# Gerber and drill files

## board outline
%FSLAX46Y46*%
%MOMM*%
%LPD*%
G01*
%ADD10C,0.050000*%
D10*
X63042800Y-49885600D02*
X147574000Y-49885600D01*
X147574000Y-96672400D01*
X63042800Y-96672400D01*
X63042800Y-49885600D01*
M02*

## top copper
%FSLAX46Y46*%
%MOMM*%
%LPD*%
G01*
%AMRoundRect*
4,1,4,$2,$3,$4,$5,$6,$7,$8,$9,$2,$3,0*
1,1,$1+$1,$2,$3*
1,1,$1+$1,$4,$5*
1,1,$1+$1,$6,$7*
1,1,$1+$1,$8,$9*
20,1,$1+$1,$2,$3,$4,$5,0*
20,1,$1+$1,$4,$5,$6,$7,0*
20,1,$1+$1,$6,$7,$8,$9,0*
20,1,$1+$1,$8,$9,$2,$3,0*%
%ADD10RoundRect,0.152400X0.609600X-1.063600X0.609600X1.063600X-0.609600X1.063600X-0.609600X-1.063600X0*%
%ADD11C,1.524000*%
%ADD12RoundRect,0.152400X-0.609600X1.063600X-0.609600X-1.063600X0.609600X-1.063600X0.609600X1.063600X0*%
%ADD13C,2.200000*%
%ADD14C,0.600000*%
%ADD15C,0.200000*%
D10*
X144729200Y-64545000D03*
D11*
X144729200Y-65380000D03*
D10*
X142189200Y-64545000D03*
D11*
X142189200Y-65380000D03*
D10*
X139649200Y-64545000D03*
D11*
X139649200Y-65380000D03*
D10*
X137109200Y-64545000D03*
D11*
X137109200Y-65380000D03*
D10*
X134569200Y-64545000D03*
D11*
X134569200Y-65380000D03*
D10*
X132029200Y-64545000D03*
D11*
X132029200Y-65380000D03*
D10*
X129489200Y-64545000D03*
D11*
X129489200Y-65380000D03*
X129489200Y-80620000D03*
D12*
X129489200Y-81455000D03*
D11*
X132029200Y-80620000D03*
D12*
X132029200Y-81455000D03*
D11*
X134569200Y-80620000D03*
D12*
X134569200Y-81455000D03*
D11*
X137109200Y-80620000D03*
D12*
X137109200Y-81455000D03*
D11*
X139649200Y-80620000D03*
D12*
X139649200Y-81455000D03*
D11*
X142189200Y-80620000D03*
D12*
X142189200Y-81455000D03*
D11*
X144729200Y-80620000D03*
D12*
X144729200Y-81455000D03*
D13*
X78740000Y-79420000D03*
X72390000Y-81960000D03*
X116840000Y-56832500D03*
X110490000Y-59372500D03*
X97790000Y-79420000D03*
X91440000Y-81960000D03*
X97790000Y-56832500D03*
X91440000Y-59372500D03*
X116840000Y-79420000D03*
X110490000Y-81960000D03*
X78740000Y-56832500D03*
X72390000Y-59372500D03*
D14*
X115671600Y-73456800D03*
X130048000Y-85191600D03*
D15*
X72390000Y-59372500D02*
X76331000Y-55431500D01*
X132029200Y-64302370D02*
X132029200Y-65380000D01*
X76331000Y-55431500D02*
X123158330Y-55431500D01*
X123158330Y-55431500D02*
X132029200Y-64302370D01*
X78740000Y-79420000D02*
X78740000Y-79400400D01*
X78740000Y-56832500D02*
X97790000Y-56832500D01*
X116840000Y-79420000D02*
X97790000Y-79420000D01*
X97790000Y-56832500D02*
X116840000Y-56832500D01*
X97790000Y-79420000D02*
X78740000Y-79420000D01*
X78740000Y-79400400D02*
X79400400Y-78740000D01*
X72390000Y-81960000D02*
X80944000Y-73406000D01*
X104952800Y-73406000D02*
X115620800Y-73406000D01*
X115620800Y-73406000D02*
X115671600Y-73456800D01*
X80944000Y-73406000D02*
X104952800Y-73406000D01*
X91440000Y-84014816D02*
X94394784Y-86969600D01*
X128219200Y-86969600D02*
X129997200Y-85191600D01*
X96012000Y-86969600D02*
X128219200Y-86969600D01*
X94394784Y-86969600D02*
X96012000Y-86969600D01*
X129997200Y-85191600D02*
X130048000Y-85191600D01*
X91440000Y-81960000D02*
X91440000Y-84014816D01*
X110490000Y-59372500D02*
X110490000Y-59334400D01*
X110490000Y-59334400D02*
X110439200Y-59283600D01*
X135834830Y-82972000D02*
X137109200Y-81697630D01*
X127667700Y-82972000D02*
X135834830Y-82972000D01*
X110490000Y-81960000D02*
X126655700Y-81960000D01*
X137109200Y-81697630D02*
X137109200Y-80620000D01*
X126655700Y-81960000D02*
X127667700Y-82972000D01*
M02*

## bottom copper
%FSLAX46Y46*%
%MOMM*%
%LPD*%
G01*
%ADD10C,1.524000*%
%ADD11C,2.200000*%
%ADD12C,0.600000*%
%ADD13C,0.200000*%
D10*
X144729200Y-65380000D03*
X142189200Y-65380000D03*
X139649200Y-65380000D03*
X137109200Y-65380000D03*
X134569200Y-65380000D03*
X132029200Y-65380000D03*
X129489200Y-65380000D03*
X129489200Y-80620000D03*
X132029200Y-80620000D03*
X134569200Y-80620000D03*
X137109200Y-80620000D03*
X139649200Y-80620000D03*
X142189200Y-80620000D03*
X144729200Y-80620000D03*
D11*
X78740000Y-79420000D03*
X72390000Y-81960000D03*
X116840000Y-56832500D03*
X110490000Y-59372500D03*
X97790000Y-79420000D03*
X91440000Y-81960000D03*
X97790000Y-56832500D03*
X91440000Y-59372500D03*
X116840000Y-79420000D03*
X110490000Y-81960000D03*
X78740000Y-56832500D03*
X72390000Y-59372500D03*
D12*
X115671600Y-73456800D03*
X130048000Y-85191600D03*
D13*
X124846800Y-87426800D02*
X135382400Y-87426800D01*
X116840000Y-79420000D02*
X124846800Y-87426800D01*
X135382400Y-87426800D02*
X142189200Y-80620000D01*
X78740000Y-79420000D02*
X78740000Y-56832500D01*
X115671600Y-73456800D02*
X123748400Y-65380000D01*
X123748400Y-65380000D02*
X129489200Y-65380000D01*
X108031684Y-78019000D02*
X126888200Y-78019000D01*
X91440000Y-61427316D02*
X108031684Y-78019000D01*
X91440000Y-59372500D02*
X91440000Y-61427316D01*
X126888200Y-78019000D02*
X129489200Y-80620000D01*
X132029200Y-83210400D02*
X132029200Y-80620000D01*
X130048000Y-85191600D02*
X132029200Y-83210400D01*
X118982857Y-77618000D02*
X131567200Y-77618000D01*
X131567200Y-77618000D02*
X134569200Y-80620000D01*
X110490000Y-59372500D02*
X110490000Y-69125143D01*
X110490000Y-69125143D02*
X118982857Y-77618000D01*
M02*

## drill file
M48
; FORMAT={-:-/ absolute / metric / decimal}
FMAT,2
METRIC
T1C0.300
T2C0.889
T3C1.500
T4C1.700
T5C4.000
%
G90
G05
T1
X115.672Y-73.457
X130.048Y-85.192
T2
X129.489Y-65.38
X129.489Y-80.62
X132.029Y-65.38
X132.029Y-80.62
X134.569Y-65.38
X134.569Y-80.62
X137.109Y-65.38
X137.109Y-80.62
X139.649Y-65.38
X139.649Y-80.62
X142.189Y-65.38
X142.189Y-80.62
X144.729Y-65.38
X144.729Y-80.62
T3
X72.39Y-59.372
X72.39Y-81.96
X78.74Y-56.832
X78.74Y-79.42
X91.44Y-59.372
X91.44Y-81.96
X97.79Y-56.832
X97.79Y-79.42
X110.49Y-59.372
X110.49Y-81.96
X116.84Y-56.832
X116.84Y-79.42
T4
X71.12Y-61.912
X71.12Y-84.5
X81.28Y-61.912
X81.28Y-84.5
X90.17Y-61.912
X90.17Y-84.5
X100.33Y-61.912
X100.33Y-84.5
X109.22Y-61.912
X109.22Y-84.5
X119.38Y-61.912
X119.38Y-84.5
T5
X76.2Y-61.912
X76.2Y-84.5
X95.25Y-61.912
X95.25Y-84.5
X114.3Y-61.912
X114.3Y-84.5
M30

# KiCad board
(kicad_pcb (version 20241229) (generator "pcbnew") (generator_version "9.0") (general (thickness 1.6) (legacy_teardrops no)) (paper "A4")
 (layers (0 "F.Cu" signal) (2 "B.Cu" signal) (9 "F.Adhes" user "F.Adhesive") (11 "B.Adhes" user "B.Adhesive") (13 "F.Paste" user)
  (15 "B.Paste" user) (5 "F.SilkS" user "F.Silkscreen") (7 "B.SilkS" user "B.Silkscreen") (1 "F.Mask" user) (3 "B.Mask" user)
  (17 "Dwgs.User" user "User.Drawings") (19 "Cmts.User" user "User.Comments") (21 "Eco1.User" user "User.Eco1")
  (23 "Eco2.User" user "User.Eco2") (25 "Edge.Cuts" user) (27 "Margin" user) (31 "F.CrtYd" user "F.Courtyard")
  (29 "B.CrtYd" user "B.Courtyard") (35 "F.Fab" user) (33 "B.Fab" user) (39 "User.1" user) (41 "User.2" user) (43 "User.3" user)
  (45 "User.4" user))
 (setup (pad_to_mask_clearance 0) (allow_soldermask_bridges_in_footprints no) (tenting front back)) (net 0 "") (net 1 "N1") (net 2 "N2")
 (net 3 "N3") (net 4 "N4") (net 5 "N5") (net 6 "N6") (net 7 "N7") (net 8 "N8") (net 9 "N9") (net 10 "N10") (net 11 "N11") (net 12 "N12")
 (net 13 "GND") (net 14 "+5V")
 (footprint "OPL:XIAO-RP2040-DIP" (layer "F.Cu") (at 137.1092 73 -90)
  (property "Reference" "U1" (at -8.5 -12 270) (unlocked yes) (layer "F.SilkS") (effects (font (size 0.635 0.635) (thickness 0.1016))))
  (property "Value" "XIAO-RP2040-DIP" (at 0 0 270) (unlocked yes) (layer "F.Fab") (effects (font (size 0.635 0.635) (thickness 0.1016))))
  (pad "1" smd roundrect (at -8.455 -7.62 90) (size 2.432 1.524) (layers "F.Cu" "F.Mask") (roundrect_rratio 0.1) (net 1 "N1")
   (thermal_bridge_angle 45))
  (pad "1" thru_hole circle (at -7.62 -7.62 90) (size 1.524 1.524) (drill 0.889) (layers "*.Cu" "*.Mask") (remove_unused_layers no)
   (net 1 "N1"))
  (pad "2" smd roundrect (at -8.455 -5.08 90) (size 2.432 1.524) (layers "F.Cu" "F.Mask") (roundrect_rratio 0.1) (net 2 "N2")
   (thermal_bridge_angle 45))
  (pad "2" thru_hole circle (at -7.62 -5.08 90) (size 1.524 1.524) (drill 0.889) (layers "*.Cu" "*.Mask") (remove_unused_layers no)
   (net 2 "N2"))
  (pad "3" smd roundrect (at -8.455 -2.54 90) (size 2.432 1.524) (layers "F.Cu" "F.Mask") (roundrect_rratio 0.1) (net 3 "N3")
   (thermal_bridge_angle 45))
  (pad "3" thru_hole circle (at -7.62 -2.54 90) (size 1.524 1.524) (drill 0.889) (layers "*.Cu" "*.Mask") (remove_unused_layers no)
   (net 3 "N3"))
  (pad "4" smd roundrect (at -8.455 0 90) (size 2.432 1.524) (layers "F.Cu" "F.Mask") (roundrect_rratio 0.1) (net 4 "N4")
   (thermal_bridge_angle 45))
  (pad "4" thru_hole circle (at -7.62 0 90) (size 1.524 1.524) (drill 0.889) (layers "*.Cu" "*.Mask") (remove_unused_layers no) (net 4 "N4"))
  (pad "5" smd roundrect (at -8.455 2.54 90) (size 2.432 1.524) (layers "F.Cu" "F.Mask") (roundrect_rratio 0.1) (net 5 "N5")
   (thermal_bridge_angle 45))
  (pad "5" thru_hole circle (at -7.62 2.54 90) (size 1.524 1.524) (drill 0.889) (layers "*.Cu" "*.Mask") (remove_unused_layers no)
   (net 5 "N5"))
  (pad "6" smd roundrect (at -8.455 5.08 90) (size 2.432 1.524) (layers "F.Cu" "F.Mask") (roundrect_rratio 0.1) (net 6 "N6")
   (thermal_bridge_angle 45))
  (pad "6" thru_hole circle (at -7.62 5.08 90) (size 1.524 1.524) (drill 0.889) (layers "*.Cu" "*.Mask") (remove_unused_layers no)
   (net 6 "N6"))
  (pad "7" smd roundrect (at -8.455 7.62 90) (size 2.432 1.524) (layers "F.Cu" "F.Mask") (roundrect_rratio 0.1) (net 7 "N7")
   (thermal_bridge_angle 45))
  (pad "7" thru_hole circle (at -7.62 7.62 90) (size 1.524 1.524) (drill 0.889) (layers "*.Cu" "*.Mask") (remove_unused_layers no)
   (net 7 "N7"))
  (pad "8" thru_hole circle (at 7.62 7.62 270) (size 1.524 1.524) (drill 0.889) (layers "*.Cu" "*.Mask") (remove_unused_layers no)
   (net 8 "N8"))
  (pad "8" smd roundrect (at 8.455 7.62 270) (size 2.432 1.524) (layers "F.Cu" "F.Mask") (roundrect_rratio 0.1) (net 8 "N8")
   (thermal_bridge_angle 45))
  (pad "9" thru_hole circle (at 7.62 5.08 270) (size 1.524 1.524) (drill 0.889) (layers "*.Cu" "*.Mask") (remove_unused_layers no)
   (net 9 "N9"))
  (pad "9" smd roundrect (at 8.455 5.08 270) (size 2.432 1.524) (layers "F.Cu" "F.Mask") (roundrect_rratio 0.1) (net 9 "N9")
   (thermal_bridge_angle 45))
  (pad "10" thru_hole circle (at 7.62 2.54 270) (size 1.524 1.524) (drill 0.889) (layers "*.Cu" "*.Mask") (remove_unused_layers no)
   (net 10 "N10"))
  (pad "10" smd roundrect (at 8.455 2.54 270) (size 2.432 1.524) (layers "F.Cu" "F.Mask") (roundrect_rratio 0.1) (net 10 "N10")
   (thermal_bridge_angle 45))
  (pad "11" thru_hole circle (at 7.62 0 270) (size 1.524 1.524) (drill 0.889) (layers "*.Cu" "*.Mask") (remove_unused_layers no)
   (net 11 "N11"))
  (pad "11" smd roundrect (at 8.455 0 270) (size 2.432 1.524) (layers "F.Cu" "F.Mask") (roundrect_rratio 0.1) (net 11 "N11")
   (thermal_bridge_angle 45))
  (pad "12" thru_hole circle (at 7.62 -2.54 270) (size 1.524 1.524) (drill 0.889) (layers "*.Cu" "*.Mask") (remove_unused_layers no)
   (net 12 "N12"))
  (pad "12" smd roundrect (at 8.455 -2.54 270) (size 2.432 1.524) (layers "F.Cu" "F.Mask") (roundrect_rratio 0.1) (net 12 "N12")
   (thermal_bridge_angle 45))
  (pad "13" thru_hole circle (at 7.62 -5.08 270) (size 1.524 1.524) (drill 0.889) (layers "*.Cu" "*.Mask") (remove_unused_layers no)
   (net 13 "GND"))
  (pad "13" smd roundrect (at 8.455 -5.08 270) (size 2.432 1.524) (layers "F.Cu" "F.Mask") (roundrect_rratio 0.1) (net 13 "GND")
   (thermal_bridge_angle 45))
  (pad "14" thru_hole circle (at 7.62 -7.62 270) (size 1.524 1.524) (drill 0.889) (layers "*.Cu" "*.Mask") (remove_unused_layers no)
   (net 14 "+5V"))
  (pad "14" smd roundrect (at 8.455 -7.62 270) (size 2.432 1.524) (layers "F.Cu" "F.Mask") (roundrect_rratio 0.1) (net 14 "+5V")
   (thermal_bridge_angle 45)))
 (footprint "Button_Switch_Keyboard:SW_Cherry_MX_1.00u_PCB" (layer "F.Cu") (at 78.74 79.42)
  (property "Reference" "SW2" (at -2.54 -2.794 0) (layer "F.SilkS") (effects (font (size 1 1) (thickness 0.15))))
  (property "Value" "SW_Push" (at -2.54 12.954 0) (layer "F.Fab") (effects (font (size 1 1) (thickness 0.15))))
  (pad "" np_thru_hole circle (at -7.62 5.08) (size 1.7 1.7) (drill 1.7) (layers "*.Cu" "*.Mask"))
  (pad "" np_thru_hole circle (at -2.54 5.08) (size 4 4) (drill 4) (layers "*.Cu" "*.Mask"))
  (pad "" np_thru_hole circle (at 2.54 5.08) (size 1.7 1.7) (drill 1.7) (layers "*.Cu" "*.Mask"))
  (pad "1" thru_hole circle (at 0 0) (size 2.2 2.2) (drill 1.5) (layers "*.Cu" "*.Mask") (remove_unused_layers no) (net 13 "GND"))
  (pad "2" thru_hole circle (at -6.35 2.54) (size 2.2 2.2) (drill 1.5) (layers "*.Cu" "*.Mask") (remove_unused_layers no) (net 7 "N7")))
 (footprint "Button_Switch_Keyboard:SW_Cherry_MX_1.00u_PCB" (layer "F.Cu") (at 116.84 56.8325)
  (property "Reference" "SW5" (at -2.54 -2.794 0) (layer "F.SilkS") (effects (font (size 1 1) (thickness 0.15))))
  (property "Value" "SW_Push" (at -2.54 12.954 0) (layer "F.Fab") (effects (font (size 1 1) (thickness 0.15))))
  (pad "" np_thru_hole circle (at -7.62 5.08) (size 1.7 1.7) (drill 1.7) (layers "*.Cu" "*.Mask"))
  (pad "" np_thru_hole circle (at -2.54 5.08) (size 4 4) (drill 4) (layers "*.Cu" "*.Mask"))
  (pad "" np_thru_hole circle (at 2.54 5.08) (size 1.7 1.7) (drill 1.7) (layers "*.Cu" "*.Mask"))
  (pad "1" thru_hole circle (at 0 0) (size 2.2 2.2) (drill 1.5) (layers "*.Cu" "*.Mask") (remove_unused_layers no) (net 13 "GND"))
  (pad "2" thru_hole circle (at -6.35 2.54) (size 2.2 2.2) (drill 1.5) (layers "*.Cu" "*.Mask") (remove_unused_layers no) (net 10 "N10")))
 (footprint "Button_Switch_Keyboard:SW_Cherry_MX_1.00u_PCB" (layer "F.Cu") (at 97.79 79.42)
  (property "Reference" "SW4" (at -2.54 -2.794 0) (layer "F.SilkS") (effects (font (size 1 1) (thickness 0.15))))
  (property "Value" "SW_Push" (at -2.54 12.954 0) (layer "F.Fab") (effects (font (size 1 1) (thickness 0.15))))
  (pad "" np_thru_hole circle (at -7.62 5.08) (size 1.7 1.7) (drill 1.7) (layers "*.Cu" "*.Mask"))
  (pad "" np_thru_hole circle (at -2.54 5.08) (size 4 4) (drill 4) (layers "*.Cu" "*.Mask"))
  (pad "" np_thru_hole circle (at 2.54 5.08) (size 1.7 1.7) (drill 1.7) (layers "*.Cu" "*.Mask"))
  (pad "1" thru_hole circle (at 0 0) (size 2.2 2.2) (drill 1.5) (layers "*.Cu" "*.Mask") (remove_unused_layers no) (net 13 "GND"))
  (pad "2" thru_hole circle (at -6.35 2.54) (size 2.2 2.2) (drill 1.5) (layers "*.Cu" "*.Mask") (remove_unused_layers no) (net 9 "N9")))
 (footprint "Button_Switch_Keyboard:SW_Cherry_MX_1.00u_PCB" (layer "F.Cu") (at 97.79 56.8325)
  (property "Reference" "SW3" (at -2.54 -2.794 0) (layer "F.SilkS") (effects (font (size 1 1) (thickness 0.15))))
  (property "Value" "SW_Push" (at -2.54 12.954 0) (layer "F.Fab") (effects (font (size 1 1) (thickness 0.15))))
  (pad "" np_thru_hole circle (at -7.62 5.08) (size 1.7 1.7) (drill 1.7) (layers "*.Cu" "*.Mask"))
  (pad "" np_thru_hole circle (at -2.54 5.08) (size 4 4) (drill 4) (layers "*.Cu" "*.Mask"))
  (pad "" np_thru_hole circle (at 2.54 5.08) (size 1.7 1.7) (drill 1.7) (layers "*.Cu" "*.Mask"))
  (pad "1" thru_hole circle (at 0 0) (size 2.2 2.2) (drill 1.5) (layers "*.Cu" "*.Mask") (remove_unused_layers no) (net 13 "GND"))
  (pad "2" thru_hole circle (at -6.35 2.54) (size 2.2 2.2) (drill 1.5) (layers "*.Cu" "*.Mask") (remove_unused_layers no) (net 8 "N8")))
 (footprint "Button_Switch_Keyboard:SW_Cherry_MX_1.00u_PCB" (layer "F.Cu") (at 116.84 79.42)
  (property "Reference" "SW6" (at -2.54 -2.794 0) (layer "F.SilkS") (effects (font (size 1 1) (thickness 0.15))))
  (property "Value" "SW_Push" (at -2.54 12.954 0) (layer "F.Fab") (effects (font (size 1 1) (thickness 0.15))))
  (pad "" np_thru_hole circle (at -7.62 5.08) (size 1.7 1.7) (drill 1.7) (layers "*.Cu" "*.Mask"))
  (pad "" np_thru_hole circle (at -2.54 5.08) (size 4 4) (drill 4) (layers "*.Cu" "*.Mask"))
  (pad "" np_thru_hole circle (at 2.54 5.08) (size 1.7 1.7) (drill 1.7) (layers "*.Cu" "*.Mask"))
  (pad "1" thru_hole circle (at 0 0) (size 2.2 2.2) (drill 1.5) (layers "*.Cu" "*.Mask") (remove_unused_layers no) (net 13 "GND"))
  (pad "2" thru_hole circle (at -6.35 2.54) (size 2.2 2.2) (drill 1.5) (layers "*.Cu" "*.Mask") (remove_unused_layers no) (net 11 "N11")))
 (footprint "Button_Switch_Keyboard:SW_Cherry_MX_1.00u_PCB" (layer "F.Cu") (at 78.74 56.8325)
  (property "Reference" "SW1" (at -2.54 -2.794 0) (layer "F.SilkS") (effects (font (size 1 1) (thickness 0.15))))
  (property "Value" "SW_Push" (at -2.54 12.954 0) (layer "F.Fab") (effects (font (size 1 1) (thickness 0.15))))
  (pad "" np_thru_hole circle (at -7.62 5.08) (size 1.7 1.7) (drill 1.7) (layers "*.Cu" "*.Mask"))
  (pad "" np_thru_hole circle (at -2.54 5.08) (size 4 4) (drill 4) (layers "*.Cu" "*.Mask"))
  (pad "" np_thru_hole circle (at 2.54 5.08) (size 1.7 1.7) (drill 1.7) (layers "*.Cu" "*.Mask"))
  (pad "1" thru_hole circle (at 0 0) (size 2.2 2.2) (drill 1.5) (layers "*.Cu" "*.Mask") (remove_unused_layers no) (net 13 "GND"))
  (pad "2" thru_hole circle (at -6.35 2.54) (size 2.2 2.2) (drill 1.5) (layers "*.Cu" "*.Mask") (remove_unused_layers no) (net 6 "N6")))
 (gr_rect (start 63.0428 49.8856) (end 147.574 96.6724) (stroke (width 0.05) (type default)) (fill no) (layer "Edge.Cuts"))
 (segment (start 72.39 59.3725) (end 76.331 55.4315) (width 0.2) (layer "F.Cu") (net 6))
 (segment (start 132.0292 64.30237) (end 132.0292 65.38) (width 0.2) (layer "F.Cu") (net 6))
 (segment (start 76.331 55.4315) (end 123.15833 55.4315) (width 0.2) (layer "F.Cu") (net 6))
 (segment (start 123.15833 55.4315) (end 132.0292 64.30237) (width 0.2) (layer "F.Cu") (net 6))
 (segment (start 78.74 79.42) (end 78.74 79.4004) (width 0.2) (layer "F.Cu") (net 13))
 (segment (start 78.74 56.8325) (end 97.79 56.8325) (width 0.2) (layer "F.Cu") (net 13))
 (segment (start 116.84 79.42) (end 97.79 79.42) (width 0.2) (layer "F.Cu") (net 13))
 (segment (start 97.79 56.8325) (end 116.84 56.8325) (width 0.2) (layer "F.Cu") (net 13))
 (segment (start 97.79 79.42) (end 78.74 79.42) (width 0.2) (layer "F.Cu") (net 13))
 (segment (start 78.74 79.4004) (end 79.4004 78.74) (width 0.2) (layer "F.Cu") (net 13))
 (segment (start 124.8468 87.4268) (end 135.3824 87.4268) (width 0.2) (layer "B.Cu") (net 13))
 (segment (start 116.84 79.42) (end 124.8468 87.4268) (width 0.2) (layer "B.Cu") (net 13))
 (segment (start 135.3824 87.4268) (end 142.1892 80.62) (width 0.2) (layer "B.Cu") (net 13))
 (segment (start 78.74 79.42) (end 78.74 56.8325) (width 0.2) (layer "B.Cu") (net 13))
 (segment (start 72.39 81.96) (end 80.944 73.406) (width 0.2) (layer "F.Cu") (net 7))
 (segment (start 104.9528 73.406) (end 115.6208 73.406) (width 0.2) (layer "F.Cu") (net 7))
 (segment (start 115.6208 73.406) (end 115.6716 73.4568) (width 0.2) (layer "F.Cu") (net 7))
 (segment (start 80.944 73.406) (end 104.9528 73.406) (width 0.2) (layer "F.Cu") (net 7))
 (via (at 115.6716 73.4568) (size 0.6) (drill 0.3) (layers "F.Cu" "B.Cu") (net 7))
 (segment (start 115.6716 73.4568) (end 123.7484 65.38) (width 0.2) (layer "B.Cu") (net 7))
 (segment (start 123.7484 65.38) (end 129.4892 65.38) (width 0.2) (layer "B.Cu") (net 7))
 (segment (start 108.031684 78.019) (end 126.8882 78.019) (width 0.2) (layer "B.Cu") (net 8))
 (segment (start 91.44 61.427316) (end 108.031684 78.019) (width 0.2) (layer "B.Cu") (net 8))
 (segment (start 91.44 59.3725) (end 91.44 61.427316) (width 0.2) (layer "B.Cu") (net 8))
 (segment (start 126.8882 78.019) (end 129.4892 80.62) (width 0.2) (layer "B.Cu") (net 8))
 (segment (start 91.44 84.014816) (end 94.394784 86.9696) (width 0.2) (layer "F.Cu") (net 9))
 (segment (start 128.2192 86.9696) (end 129.9972 85.1916) (width 0.2) (layer "F.Cu") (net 9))
 (segment (start 96.012 86.9696) (end 128.2192 86.9696) (width 0.2) (layer "F.Cu") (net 9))
 (segment (start 94.394784 86.9696) (end 96.012 86.9696) (width 0.2) (layer "F.Cu") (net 9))
 (segment (start 129.9972 85.1916) (end 130.048 85.1916) (width 0.2) (layer "F.Cu") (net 9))
 (segment (start 91.44 81.96) (end 91.44 84.014816) (width 0.2) (layer "F.Cu") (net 9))
 (via (at 130.048 85.1916) (size 0.6) (drill 0.3) (layers "F.Cu" "B.Cu") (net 9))
 (segment (start 132.0292 83.2104) (end 132.0292 80.62) (width 0.2) (layer "B.Cu") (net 9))
 (segment (start 130.048 85.1916) (end 132.0292 83.2104) (width 0.2) (layer "B.Cu") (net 9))
 (segment (start 110.49 59.3725) (end 110.49 59.3344) (width 0.2) (layer "F.Cu") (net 10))
 (segment (start 110.49 59.3344) (end 110.4392 59.2836) (width 0.2) (layer "F.Cu") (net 10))
 (segment (start 118.982857 77.618) (end 131.5672 77.618) (width 0.2) (layer "B.Cu") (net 10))
 (segment (start 131.5672 77.618) (end 134.5692 80.62) (width 0.2) (layer "B.Cu") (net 10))
 (segment (start 110.49 59.3725) (end 110.49 69.125143) (width 0.2) (layer "B.Cu") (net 10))
 (segment (start 110.49 69.125143) (end 118.982857 77.618) (width 0.2) (layer "B.Cu") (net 10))
 (segment (start 135.83483 82.972) (end 137.1092 81.69763) (width 0.2) (layer "F.Cu") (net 11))
 (segment (start 127.6677 82.972) (end 135.83483 82.972) (width 0.2) (layer "F.Cu") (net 11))
 (segment (start 110.49 81.96) (end 126.6557 81.96) (width 0.2) (layer "F.Cu") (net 11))
 (segment (start 137.1092 81.69763) (end 137.1092 80.62) (width 0.2) (layer "F.Cu") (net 11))
 (segment (start 126.6557 81.96) (end 127.6677 82.972) (width 0.2) (layer "F.Cu") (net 11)))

